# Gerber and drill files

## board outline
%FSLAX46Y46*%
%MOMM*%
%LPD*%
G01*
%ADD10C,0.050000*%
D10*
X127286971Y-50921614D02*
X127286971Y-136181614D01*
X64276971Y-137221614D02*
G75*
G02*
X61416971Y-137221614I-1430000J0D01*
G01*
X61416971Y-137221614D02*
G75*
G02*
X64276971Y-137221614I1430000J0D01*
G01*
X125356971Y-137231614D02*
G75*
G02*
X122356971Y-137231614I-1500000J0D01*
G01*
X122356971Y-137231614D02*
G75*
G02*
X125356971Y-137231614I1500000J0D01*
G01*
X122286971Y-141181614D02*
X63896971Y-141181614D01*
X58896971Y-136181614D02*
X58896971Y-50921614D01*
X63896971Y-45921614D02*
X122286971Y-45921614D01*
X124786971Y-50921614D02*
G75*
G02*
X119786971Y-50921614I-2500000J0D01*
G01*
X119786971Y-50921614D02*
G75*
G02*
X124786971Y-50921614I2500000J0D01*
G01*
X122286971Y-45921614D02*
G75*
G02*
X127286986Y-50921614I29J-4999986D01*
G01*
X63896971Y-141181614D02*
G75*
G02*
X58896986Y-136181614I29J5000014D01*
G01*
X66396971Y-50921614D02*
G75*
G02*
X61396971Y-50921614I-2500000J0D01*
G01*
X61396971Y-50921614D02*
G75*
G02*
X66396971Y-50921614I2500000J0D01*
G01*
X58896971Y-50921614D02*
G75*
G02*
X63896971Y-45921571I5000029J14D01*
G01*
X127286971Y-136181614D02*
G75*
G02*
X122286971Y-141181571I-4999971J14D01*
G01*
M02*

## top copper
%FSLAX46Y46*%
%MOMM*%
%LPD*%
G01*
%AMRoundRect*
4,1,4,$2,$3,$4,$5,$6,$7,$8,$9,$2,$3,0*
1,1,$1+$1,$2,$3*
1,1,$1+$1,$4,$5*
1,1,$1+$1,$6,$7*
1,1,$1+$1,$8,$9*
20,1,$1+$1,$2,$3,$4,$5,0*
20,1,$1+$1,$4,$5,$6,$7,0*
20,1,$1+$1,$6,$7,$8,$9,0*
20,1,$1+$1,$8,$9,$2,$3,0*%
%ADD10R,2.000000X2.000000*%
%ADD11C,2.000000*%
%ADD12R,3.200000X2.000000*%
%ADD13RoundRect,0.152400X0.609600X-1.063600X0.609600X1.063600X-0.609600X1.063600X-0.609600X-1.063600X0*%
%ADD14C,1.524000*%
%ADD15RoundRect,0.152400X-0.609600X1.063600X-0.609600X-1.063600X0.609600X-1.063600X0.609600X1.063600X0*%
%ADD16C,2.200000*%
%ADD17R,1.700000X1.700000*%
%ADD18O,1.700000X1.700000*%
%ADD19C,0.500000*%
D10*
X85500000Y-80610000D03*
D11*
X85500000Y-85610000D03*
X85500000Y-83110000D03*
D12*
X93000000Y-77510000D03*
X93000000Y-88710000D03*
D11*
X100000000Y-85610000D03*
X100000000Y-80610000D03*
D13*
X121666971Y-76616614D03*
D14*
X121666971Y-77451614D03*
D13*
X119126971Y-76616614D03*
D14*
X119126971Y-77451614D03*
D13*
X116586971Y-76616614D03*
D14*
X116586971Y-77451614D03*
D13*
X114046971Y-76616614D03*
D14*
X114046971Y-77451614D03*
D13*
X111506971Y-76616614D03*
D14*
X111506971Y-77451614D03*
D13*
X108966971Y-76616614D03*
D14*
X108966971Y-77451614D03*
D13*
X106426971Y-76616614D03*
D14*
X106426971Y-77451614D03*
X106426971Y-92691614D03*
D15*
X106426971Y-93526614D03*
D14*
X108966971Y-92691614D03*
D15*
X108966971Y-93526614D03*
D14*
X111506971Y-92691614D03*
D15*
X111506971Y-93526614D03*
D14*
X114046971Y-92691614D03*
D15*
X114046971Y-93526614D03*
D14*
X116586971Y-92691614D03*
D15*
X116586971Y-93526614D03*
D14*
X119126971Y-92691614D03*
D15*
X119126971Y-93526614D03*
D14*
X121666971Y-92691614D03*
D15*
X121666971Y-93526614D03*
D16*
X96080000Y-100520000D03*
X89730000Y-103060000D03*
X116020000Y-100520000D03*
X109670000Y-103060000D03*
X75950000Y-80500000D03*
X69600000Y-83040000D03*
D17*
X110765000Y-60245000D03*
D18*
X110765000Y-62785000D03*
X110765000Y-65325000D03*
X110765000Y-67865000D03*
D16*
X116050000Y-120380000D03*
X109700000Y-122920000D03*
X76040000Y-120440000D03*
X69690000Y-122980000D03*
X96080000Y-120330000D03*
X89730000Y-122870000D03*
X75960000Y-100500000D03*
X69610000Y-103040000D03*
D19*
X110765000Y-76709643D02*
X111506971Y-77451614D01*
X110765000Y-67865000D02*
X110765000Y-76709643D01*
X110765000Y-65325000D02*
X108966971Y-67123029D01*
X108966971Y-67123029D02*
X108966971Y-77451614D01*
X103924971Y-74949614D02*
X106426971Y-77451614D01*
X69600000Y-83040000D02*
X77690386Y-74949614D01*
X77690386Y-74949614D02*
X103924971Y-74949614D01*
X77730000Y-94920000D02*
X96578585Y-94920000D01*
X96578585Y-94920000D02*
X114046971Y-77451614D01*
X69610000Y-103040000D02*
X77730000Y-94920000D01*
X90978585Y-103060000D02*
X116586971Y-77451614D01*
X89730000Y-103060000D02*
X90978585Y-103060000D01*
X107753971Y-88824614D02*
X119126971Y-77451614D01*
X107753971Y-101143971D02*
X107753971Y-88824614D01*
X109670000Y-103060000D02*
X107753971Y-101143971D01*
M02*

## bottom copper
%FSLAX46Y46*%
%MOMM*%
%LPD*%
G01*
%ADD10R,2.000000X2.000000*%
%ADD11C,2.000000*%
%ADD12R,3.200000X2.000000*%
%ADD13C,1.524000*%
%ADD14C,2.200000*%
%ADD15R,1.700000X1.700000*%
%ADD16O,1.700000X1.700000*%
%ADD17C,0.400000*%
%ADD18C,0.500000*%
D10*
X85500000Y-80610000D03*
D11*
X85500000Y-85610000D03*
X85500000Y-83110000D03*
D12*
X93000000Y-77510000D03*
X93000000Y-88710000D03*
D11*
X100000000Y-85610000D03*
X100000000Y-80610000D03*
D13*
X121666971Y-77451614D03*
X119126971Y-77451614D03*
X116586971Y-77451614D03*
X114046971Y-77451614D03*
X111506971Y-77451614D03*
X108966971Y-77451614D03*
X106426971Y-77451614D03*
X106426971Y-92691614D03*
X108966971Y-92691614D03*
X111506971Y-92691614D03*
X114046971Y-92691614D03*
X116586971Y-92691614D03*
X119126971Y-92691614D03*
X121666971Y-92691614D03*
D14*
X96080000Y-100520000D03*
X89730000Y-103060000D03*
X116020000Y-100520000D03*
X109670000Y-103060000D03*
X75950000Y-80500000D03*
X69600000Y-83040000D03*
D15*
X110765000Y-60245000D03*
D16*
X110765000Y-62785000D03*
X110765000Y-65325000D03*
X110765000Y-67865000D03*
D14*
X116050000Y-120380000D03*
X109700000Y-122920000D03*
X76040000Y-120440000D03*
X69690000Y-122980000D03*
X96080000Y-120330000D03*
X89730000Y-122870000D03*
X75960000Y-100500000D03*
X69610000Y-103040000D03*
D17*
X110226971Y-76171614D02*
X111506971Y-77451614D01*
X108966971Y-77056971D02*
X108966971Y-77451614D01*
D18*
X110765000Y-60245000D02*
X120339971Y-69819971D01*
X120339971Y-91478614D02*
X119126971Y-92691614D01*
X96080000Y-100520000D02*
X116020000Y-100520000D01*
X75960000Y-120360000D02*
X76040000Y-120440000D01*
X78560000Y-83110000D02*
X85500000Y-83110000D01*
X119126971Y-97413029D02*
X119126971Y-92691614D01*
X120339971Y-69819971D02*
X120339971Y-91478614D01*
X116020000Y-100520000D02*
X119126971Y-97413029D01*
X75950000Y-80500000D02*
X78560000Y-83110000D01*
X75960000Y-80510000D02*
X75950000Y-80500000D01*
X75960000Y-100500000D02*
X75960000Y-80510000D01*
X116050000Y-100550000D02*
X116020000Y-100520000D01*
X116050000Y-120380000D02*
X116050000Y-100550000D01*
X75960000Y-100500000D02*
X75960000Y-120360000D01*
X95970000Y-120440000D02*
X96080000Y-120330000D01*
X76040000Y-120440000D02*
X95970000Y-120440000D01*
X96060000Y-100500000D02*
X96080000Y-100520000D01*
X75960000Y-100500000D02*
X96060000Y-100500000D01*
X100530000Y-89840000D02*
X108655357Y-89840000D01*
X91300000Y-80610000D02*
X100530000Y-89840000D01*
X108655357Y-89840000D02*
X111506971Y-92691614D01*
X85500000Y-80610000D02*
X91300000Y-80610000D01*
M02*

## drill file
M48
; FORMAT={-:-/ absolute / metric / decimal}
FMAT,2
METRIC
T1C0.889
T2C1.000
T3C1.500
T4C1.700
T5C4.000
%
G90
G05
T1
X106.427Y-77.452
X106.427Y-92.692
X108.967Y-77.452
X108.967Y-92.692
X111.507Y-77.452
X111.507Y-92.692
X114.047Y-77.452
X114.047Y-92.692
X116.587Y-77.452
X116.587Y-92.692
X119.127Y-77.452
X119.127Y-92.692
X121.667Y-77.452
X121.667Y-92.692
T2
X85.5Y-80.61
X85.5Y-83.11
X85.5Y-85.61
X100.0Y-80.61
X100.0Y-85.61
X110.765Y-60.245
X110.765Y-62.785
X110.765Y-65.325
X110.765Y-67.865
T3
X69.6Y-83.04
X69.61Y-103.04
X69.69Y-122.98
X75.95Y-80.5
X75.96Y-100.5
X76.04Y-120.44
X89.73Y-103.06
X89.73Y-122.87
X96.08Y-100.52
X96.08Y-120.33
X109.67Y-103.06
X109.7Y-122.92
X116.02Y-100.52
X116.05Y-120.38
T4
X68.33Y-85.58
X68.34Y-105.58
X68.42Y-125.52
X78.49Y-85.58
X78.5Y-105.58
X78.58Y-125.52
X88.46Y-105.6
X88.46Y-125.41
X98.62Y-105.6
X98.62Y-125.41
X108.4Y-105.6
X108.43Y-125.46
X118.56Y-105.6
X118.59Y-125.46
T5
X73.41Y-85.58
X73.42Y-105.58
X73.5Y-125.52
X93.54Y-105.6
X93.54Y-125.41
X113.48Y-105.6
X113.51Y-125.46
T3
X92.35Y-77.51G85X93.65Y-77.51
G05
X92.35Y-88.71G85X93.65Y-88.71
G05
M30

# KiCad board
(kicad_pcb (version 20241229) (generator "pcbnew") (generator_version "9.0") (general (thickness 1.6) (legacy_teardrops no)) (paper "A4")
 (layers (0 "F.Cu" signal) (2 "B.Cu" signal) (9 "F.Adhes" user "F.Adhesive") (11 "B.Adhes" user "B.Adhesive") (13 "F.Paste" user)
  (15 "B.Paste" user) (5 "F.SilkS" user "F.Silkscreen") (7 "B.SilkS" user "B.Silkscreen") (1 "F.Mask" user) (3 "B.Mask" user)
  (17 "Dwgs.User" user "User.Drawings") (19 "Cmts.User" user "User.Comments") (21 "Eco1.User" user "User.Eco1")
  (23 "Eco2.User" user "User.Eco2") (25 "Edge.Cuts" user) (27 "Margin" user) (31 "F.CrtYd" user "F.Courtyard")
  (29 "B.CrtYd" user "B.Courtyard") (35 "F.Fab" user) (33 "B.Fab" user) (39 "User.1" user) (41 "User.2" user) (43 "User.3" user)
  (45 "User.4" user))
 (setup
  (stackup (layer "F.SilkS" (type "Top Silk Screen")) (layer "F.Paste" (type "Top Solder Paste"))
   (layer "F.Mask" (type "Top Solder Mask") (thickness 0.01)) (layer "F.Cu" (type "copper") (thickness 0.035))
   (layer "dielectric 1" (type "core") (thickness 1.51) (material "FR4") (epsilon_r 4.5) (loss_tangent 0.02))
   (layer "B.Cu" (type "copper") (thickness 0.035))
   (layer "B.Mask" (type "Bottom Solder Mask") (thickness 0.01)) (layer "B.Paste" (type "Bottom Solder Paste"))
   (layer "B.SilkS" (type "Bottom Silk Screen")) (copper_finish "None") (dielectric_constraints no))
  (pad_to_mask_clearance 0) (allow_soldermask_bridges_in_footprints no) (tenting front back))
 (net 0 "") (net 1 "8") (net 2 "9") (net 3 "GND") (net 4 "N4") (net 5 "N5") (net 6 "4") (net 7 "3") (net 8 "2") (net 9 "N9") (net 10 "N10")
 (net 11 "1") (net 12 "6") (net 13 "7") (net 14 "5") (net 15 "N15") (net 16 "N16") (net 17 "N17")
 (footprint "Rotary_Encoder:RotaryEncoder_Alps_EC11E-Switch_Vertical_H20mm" (layer "F.Cu") (at 85.5 80.61)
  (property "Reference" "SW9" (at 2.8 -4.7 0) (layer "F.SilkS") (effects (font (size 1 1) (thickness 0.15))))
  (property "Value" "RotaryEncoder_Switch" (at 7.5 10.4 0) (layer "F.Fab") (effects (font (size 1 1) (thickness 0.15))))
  (pad "A" thru_hole rect (at 0 0) (size 2 2) (drill 1) (layers "*.Cu" "*.Mask") (remove_unused_layers no) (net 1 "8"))
  (pad "B" thru_hole circle (at 0 5) (size 2 2) (drill 1) (layers "*.Cu" "*.Mask") (remove_unused_layers no) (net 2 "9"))
  (pad "C" thru_hole circle (at 0 2.5) (size 2 2) (drill 1) (layers "*.Cu" "*.Mask") (remove_unused_layers no) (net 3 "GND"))
  (pad "MP" thru_hole rect (at 7.5 -3.1) (size 3.2 2) (drill oval 2.8 1.5) (layers "*.Cu" "*.Mask") (remove_unused_layers no))
  (pad "MP" thru_hole rect (at 7.5 8.1) (size 3.2 2) (drill oval 2.8 1.5) (layers "*.Cu" "*.Mask") (remove_unused_layers no))
  (pad "S1" thru_hole circle (at 14.5 5) (size 2 2) (drill 1) (layers "*.Cu" "*.Mask") (remove_unused_layers no) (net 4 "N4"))
  (pad "S2" thru_hole circle (at 14.5 0) (size 2 2) (drill 1) (layers "*.Cu" "*.Mask") (remove_unused_layers no) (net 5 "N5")))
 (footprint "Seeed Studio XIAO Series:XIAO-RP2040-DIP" (layer "F.Cu") (at 114.046971 85.071614 -90)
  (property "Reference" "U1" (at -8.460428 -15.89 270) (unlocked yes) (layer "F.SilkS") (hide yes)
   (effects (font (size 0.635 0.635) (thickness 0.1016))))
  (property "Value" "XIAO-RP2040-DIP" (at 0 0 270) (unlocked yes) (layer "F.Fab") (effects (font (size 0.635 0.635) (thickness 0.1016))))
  (pad "1" smd roundrect (at -8.455 -7.62 90) (size 2.432 1.524) (layers "F.Cu" "F.Mask") (roundrect_rratio 0.1) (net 2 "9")
   (thermal_bridge_angle 45))
  (pad "1" thru_hole circle (at -7.62 -7.62 90) (size 1.524 1.524) (drill 0.889) (layers "*.Cu" "*.Mask") (remove_unused_layers no)
   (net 2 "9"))
  (pad "2" smd roundrect (at -8.455 -5.08 90) (size 2.432 1.524) (layers "F.Cu" "F.Mask") (roundrect_rratio 0.1) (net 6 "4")
   (thermal_bridge_angle 45))
  (pad "2" thru_hole circle (at -7.62 -5.08 90) (size 1.524 1.524) (drill 0.889) (layers "*.Cu" "*.Mask") (remove_unused_layers no)
   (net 6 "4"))
  (pad "3" smd roundrect (at -8.455 -2.54 90) (size 2.432 1.524) (layers "F.Cu" "F.Mask") (roundrect_rratio 0.1) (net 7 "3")
   (thermal_bridge_angle 45))
  (pad "3" thru_hole circle (at -7.62 -2.54 90) (size 1.524 1.524) (drill 0.889) (layers "*.Cu" "*.Mask") (remove_unused_layers no)
   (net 7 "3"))
  (pad "4" smd roundrect (at -8.455 0 90) (size 2.432 1.524) (layers "F.Cu" "F.Mask") (roundrect_rratio 0.1) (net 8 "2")
   (thermal_bridge_angle 45))
  (pad "4" thru_hole circle (at -7.62 0 90) (size 1.524 1.524) (drill 0.889) (layers "*.Cu" "*.Mask") (remove_unused_layers no) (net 8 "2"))
  (pad "5" smd roundrect (at -8.455 2.54 90) (size 2.432 1.524) (layers "F.Cu" "F.Mask") (roundrect_rratio 0.1) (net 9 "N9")
   (thermal_bridge_angle 45))
  (pad "5" thru_hole circle (at -7.62 2.54 90) (size 1.524 1.524) (drill 0.889) (layers "*.Cu" "*.Mask") (remove_unused_layers no)
   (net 9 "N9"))
  (pad "6" smd roundrect (at -8.455 5.08 90) (size 2.432 1.524) (layers "F.Cu" "F.Mask") (roundrect_rratio 0.1) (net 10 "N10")
   (thermal_bridge_angle 45))
  (pad "6" thru_hole circle (at -7.62 5.08 90) (size 1.524 1.524) (drill 0.889) (layers "*.Cu" "*.Mask") (remove_unused_layers no)
   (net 10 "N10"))
  (pad "7" smd roundrect (at -8.455 7.62 90) (size 2.432 1.524) (layers "F.Cu" "F.Mask") (roundrect_rratio 0.1) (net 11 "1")
   (thermal_bridge_angle 45))
  (pad "7" thru_hole circle (at -7.62 7.62 90) (size 1.524 1.524) (drill 0.889) (layers "*.Cu" "*.Mask") (remove_unused_layers no)
   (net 11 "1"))
  (pad "8" thru_hole circle (at 7.62 7.62 270) (size 1.524 1.524) (drill 0.889) (layers "*.Cu" "*.Mask") (remove_unused_layers no)
   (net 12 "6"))
  (pad "8" smd roundrect (at 8.455 7.62 270) (size 2.432 1.524) (layers "F.Cu" "F.Mask") (roundrect_rratio 0.1) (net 12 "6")
   (thermal_bridge_angle 45))
  (pad "9" thru_hole circle (at 7.62 5.08 270) (size 1.524 1.524) (drill 0.889) (layers "*.Cu" "*.Mask") (remove_unused_layers no)
   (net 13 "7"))
  (pad "9" smd roundrect (at 8.455 5.08 270) (size 2.432 1.524) (layers "F.Cu" "F.Mask") (roundrect_rratio 0.1) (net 13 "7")
   (thermal_bridge_angle 45))
  (pad "10" thru_hole circle (at 7.62 2.54 270) (size 1.524 1.524) (drill 0.889) (layers "*.Cu" "*.Mask") (remove_unused_layers no)
   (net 1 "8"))
  (pad "10" smd roundrect (at 8.455 2.54 270) (size 2.432 1.524) (layers "F.Cu" "F.Mask") (roundrect_rratio 0.1) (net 1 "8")
   (thermal_bridge_angle 45))
  (pad "11" thru_hole circle (at 7.62 0 270) (size 1.524 1.524) (drill 0.889) (layers "*.Cu" "*.Mask") (remove_unused_layers no)
   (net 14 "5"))
  (pad "11" smd roundrect (at 8.455 0 270) (size 2.432 1.524) (layers "F.Cu" "F.Mask") (roundrect_rratio 0.1) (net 14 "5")
   (thermal_bridge_angle 45))
  (pad "12" thru_hole circle (at 7.62 -2.54 270) (size 1.524 1.524) (drill 0.889) (layers "*.Cu" "*.Mask") (remove_unused_layers no)
   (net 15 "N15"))
  (pad "12" smd roundrect (at 8.455 -2.54 270) (size 2.432 1.524) (layers "F.Cu" "F.Mask") (roundrect_rratio 0.1) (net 15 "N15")
   (thermal_bridge_angle 45))
  (pad "13" thru_hole circle (at 7.62 -5.08 270) (size 1.524 1.524) (drill 0.889) (layers "*.Cu" "*.Mask") (remove_unused_layers no)
   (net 3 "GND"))
  (pad "13" smd roundrect (at 8.455 -5.08 270) (size 2.432 1.524) (layers "F.Cu" "F.Mask") (roundrect_rratio 0.1) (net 3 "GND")
   (thermal_bridge_angle 45))
  (pad "14" thru_hole circle (at 7.62 -7.62 270) (size 1.524 1.524) (drill 0.889) (layers "*.Cu" "*.Mask") (remove_unused_layers no)
   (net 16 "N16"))
  (pad "14" smd roundrect (at 8.455 -7.62 270) (size 2.432 1.524) (layers "F.Cu" "F.Mask") (roundrect_rratio 0.1) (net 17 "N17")
   (thermal_bridge_angle 45)))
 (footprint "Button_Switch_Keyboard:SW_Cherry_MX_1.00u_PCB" (layer "F.Cu") (at 96.08 100.52)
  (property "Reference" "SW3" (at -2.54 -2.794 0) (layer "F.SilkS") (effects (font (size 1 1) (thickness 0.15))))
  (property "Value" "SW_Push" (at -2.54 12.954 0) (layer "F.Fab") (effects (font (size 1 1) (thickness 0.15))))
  (pad "" np_thru_hole circle (at -7.62 5.08) (size 1.7 1.7) (drill 1.7) (layers "*.Cu" "*.Mask"))
  (pad "" np_thru_hole circle (at -2.54 5.08) (size 4 4) (drill 4) (layers "*.Cu" "*.Mask"))
  (pad "" np_thru_hole circle (at 2.54 5.08) (size 1.7 1.7) (drill 1.7) (layers "*.Cu" "*.Mask"))
  (pad "1" thru_hole circle (at 0 0) (size 2.2 2.2) (drill 1.5) (layers "*.Cu" "*.Mask") (remove_unused_layers no) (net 3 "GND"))
  (pad "2" thru_hole circle (at -6.35 2.54) (size 2.2 2.2) (drill 1.5) (layers "*.Cu" "*.Mask") (remove_unused_layers no) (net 7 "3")))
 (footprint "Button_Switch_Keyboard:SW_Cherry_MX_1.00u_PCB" (layer "F.Cu") (at 116.02 100.52)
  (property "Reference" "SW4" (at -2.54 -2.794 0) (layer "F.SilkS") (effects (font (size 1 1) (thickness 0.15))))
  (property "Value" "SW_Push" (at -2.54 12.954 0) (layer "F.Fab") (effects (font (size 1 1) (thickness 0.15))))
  (pad "" np_thru_hole circle (at -7.62 5.08) (size 1.7 1.7) (drill 1.7) (layers "*.Cu" "*.Mask"))
  (pad "" np_thru_hole circle (at -2.54 5.08) (size 4 4) (drill 4) (layers "*.Cu" "*.Mask"))
  (pad "" np_thru_hole circle (at 2.54 5.08) (size 1.7 1.7) (drill 1.7) (layers "*.Cu" "*.Mask"))
  (pad "1" thru_hole circle (at 0 0) (size 2.2 2.2) (drill 1.5) (layers "*.Cu" "*.Mask") (remove_unused_layers no) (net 3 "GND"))
  (pad "2" thru_hole circle (at -6.35 2.54) (size 2.2 2.2) (drill 1.5) (layers "*.Cu" "*.Mask") (remove_unused_layers no) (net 6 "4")))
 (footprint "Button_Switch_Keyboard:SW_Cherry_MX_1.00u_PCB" (layer "F.Cu") (at 75.95 80.5)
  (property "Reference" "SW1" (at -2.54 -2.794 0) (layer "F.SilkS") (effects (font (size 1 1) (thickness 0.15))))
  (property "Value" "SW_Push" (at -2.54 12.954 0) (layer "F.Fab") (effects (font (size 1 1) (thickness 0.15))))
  (pad "" np_thru_hole circle (at -7.62 5.08) (size 1.7 1.7) (drill 1.7) (layers "*.Cu" "*.Mask"))
  (pad "" np_thru_hole circle (at -2.54 5.08) (size 4 4) (drill 4) (layers "*.Cu" "*.Mask"))
  (pad "" np_thru_hole circle (at 2.54 5.08) (size 1.7 1.7) (drill 1.7) (layers "*.Cu" "*.Mask"))
  (pad "1" thru_hole circle (at 0 0) (size 2.2 2.2) (drill 1.5) (layers "*.Cu" "*.Mask") (remove_unused_layers no) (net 3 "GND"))
  (pad "2" thru_hole circle (at -6.35 2.54) (size 2.2 2.2) (drill 1.5) (layers "*.Cu" "*.Mask") (remove_unused_layers no) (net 11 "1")))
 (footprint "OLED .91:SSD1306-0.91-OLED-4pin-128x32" (layer "F.Cu") (at 74.265 58.055)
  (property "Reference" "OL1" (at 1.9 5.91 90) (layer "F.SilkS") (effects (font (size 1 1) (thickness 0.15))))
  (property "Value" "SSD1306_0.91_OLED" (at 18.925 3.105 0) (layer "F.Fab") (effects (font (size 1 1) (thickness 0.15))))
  (pad "1" thru_hole rect (at 36.5 2.19) (size 1.7 1.7) (drill 1) (layers "*.Cu" "*.Mask") (remove_unused_layers no) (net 3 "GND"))
  (pad "2" thru_hole oval (at 36.5 4.73) (size 1.7 1.7) (drill 1) (layers "*.Cu" "*.Mask") (remove_unused_layers no) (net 15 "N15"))
  (pad "3" thru_hole oval (at 36.5 7.27) (size 1.7 1.7) (drill 1) (layers "*.Cu" "*.Mask") (remove_unused_layers no) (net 10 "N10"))
  (pad "4" thru_hole oval (at 36.5 9.81) (size 1.7 1.7) (drill 1) (layers "*.Cu" "*.Mask") (remove_unused_layers no) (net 9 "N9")))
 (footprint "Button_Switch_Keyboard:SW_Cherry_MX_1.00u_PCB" (layer "F.Cu") (at 116.05 120.38)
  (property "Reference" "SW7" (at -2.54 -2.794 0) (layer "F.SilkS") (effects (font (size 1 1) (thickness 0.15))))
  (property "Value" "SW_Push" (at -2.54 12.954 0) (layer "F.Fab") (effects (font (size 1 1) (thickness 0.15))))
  (pad "" np_thru_hole circle (at -7.62 5.08) (size 1.7 1.7) (drill 1.7) (layers "*.Cu" "*.Mask"))
  (pad "" np_thru_hole circle (at -2.54 5.08) (size 4 4) (drill 4) (layers "*.Cu" "*.Mask"))
  (pad "" np_thru_hole circle (at 2.54 5.08) (size 1.7 1.7) (drill 1.7) (layers "*.Cu" "*.Mask"))
  (pad "1" thru_hole circle (at 0 0) (size 2.2 2.2) (drill 1.5) (layers "*.Cu" "*.Mask") (remove_unused_layers no) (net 3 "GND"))
  (pad "2" thru_hole circle (at -6.35 2.54) (size 2.2 2.2) (drill 1.5) (layers "*.Cu" "*.Mask") (remove_unused_layers no) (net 13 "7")))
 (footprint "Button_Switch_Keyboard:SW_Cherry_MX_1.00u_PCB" (layer "F.Cu") (at 76.04 120.44)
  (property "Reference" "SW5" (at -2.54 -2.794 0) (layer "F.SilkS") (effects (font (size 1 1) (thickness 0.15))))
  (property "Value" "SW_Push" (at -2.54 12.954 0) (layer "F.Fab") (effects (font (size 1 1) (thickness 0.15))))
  (pad "" np_thru_hole circle (at -7.62 5.08) (size 1.7 1.7) (drill 1.7) (layers "*.Cu" "*.Mask"))
  (pad "" np_thru_hole circle (at -2.54 5.08) (size 4 4) (drill 4) (layers "*.Cu" "*.Mask"))
  (pad "" np_thru_hole circle (at 2.54 5.08) (size 1.7 1.7) (drill 1.7) (layers "*.Cu" "*.Mask"))
  (pad "1" thru_hole circle (at 0 0) (size 2.2 2.2) (drill 1.5) (layers "*.Cu" "*.Mask") (remove_unused_layers no) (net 3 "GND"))
  (pad "2" thru_hole circle (at -6.35 2.54) (size 2.2 2.2) (drill 1.5) (layers "*.Cu" "*.Mask") (remove_unused_layers no) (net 14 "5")))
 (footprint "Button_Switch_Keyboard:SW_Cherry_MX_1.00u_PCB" (layer "F.Cu") (at 96.08 120.33)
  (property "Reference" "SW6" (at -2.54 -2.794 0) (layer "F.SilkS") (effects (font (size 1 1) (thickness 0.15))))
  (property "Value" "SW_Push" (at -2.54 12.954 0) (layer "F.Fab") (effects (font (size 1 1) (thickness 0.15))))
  (pad "" np_thru_hole circle (at -7.62 5.08) (size 1.7 1.7) (drill 1.7) (layers "*.Cu" "*.Mask"))
  (pad "" np_thru_hole circle (at -2.54 5.08) (size 4 4) (drill 4) (layers "*.Cu" "*.Mask"))
  (pad "" np_thru_hole circle (at 2.54 5.08) (size 1.7 1.7) (drill 1.7) (layers "*.Cu" "*.Mask"))
  (pad "1" thru_hole circle (at 0 0) (size 2.2 2.2) (drill 1.5) (layers "*.Cu" "*.Mask") (remove_unused_layers no) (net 3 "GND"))
  (pad "2" thru_hole circle (at -6.35 2.54) (size 2.2 2.2) (drill 1.5) (layers "*.Cu" "*.Mask") (remove_unused_layers no) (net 12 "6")))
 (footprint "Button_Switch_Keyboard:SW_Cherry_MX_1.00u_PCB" (layer "F.Cu") (at 75.96 100.5)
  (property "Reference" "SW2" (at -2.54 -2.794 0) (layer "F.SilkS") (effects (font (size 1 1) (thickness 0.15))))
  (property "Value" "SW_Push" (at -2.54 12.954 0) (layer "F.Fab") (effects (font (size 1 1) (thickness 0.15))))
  (pad "" np_thru_hole circle (at -7.62 5.08) (size 1.7 1.7) (drill 1.7) (layers "*.Cu" "*.Mask"))
  (pad "" np_thru_hole circle (at -2.54 5.08) (size 4 4) (drill 4) (layers "*.Cu" "*.Mask"))
  (pad "" np_thru_hole circle (at 2.54 5.08) (size 1.7 1.7) (drill 1.7) (layers "*.Cu" "*.Mask"))
  (pad "1" thru_hole circle (at 0 0) (size 2.2 2.2) (drill 1.5) (layers "*.Cu" "*.Mask") (remove_unused_layers no) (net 3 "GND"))
  (pad "2" thru_hole circle (at -6.35 2.54) (size 2.2 2.2) (drill 1.5) (layers "*.Cu" "*.Mask") (remove_unused_layers no) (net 8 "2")))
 (gr_line (start 127.286971 50.921614) (end 127.286971 136.181614) (stroke (width 0.05) (type default)) (layer "Edge.Cuts"))
 (gr_circle (center 62.846971 137.221614) (end 64.276971 137.221614) (stroke (width 0.05) (type solid)) (fill no) (layer "Edge.Cuts"))
 (gr_circle (center 123.856971 137.231614) (end 125.356971 137.231614) (stroke (width 0.05) (type solid)) (fill no) (layer "Edge.Cuts"))
 (gr_line (start 122.286971 141.181614) (end 63.896971 141.181614) (stroke (width 0.05) (type default)) (layer "Edge.Cuts"))
 (gr_line (start 58.896971 136.181614) (end 58.896971 50.921614) (stroke (width 0.05) (type default)) (layer "Edge.Cuts"))
 (gr_line (start 63.896971 45.921614) (end 122.286971 45.921614) (stroke (width 0.05) (type default)) (layer "Edge.Cuts"))
 (gr_circle (center 122.286971 50.921614) (end 124.786971 50.921614) (stroke (width 0.05) (type solid)) (fill no) (layer "Edge.Cuts"))
 (gr_arc (start 122.286971 45.921614) (mid 125.822505 47.38608) (end 127.286971 50.921614) (stroke (width 0.05) (type default))
  (layer "Edge.Cuts"))
 (gr_arc (start 63.896971 141.181614) (mid 60.361437 139.717148) (end 58.896971 136.181614) (stroke (width 0.05) (type default))
  (layer "Edge.Cuts"))
 (gr_circle (center 63.896971 50.921614) (end 66.396971 50.921614) (stroke (width 0.05) (type solid)) (fill no) (layer "Edge.Cuts"))
 (gr_arc (start 58.896971 50.921614) (mid 60.361437 47.38608) (end 63.896971 45.921614) (stroke (width 0.05) (type default))
  (layer "Edge.Cuts"))
 (gr_arc (start 127.286971 136.181614) (mid 125.822505 139.717148) (end 122.286971 141.181614) (stroke (width 0.05) (type default))
  (layer "Edge.Cuts"))
 (segment (start 110.765 76.709643) (end 111.506971 77.451614) (width 0.5) (layer "F.Cu") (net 9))
 (segment (start 110.765 67.865) (end 110.765 76.709643) (width 0.5) (layer "F.Cu") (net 9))
 (segment (start 110.226971 76.171614) (end 111.506971 77.451614) (width 0.4) (layer "B.Cu") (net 9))
 (segment (start 110.765 65.325) (end 108.966971 67.123029) (width 0.5) (layer "F.Cu") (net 10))
 (segment (start 108.966971 67.123029) (end 108.966971 77.451614) (width 0.5) (layer "F.Cu") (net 10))
 (segment (start 108.966971 77.056971) (end 108.966971 77.451614) (width 0.4) (layer "B.Cu") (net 10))
 (segment (start 110.765 60.245) (end 120.339971 69.819971) (width 0.5) (layer "B.Cu") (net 3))
 (segment (start 120.339971 91.478614) (end 119.126971 92.691614) (width 0.5) (layer "B.Cu") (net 3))
 (segment (start 96.08 100.52) (end 116.02 100.52) (width 0.5) (layer "B.Cu") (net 3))
 (segment (start 75.96 120.36) (end 76.04 120.44) (width 0.5) (layer "B.Cu") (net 3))
 (segment (start 78.56 83.11) (end 85.5 83.11) (width 0.5) (layer "B.Cu") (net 3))
 (segment (start 119.126971 97.413029) (end 119.126971 92.691614) (width 0.5) (layer "B.Cu") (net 3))
 (segment (start 120.339971 69.819971) (end 120.339971 91.478614) (width 0.5) (layer "B.Cu") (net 3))
 (segment (start 116.02 100.52) (end 119.126971 97.413029) (width 0.5) (layer "B.Cu") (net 3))
 (segment (start 75.95 80.5) (end 78.56 83.11) (width 0.5) (layer "B.Cu") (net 3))
 (segment (start 75.96 80.51) (end 75.95 80.5) (width 0.5) (layer "B.Cu") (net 3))
 (segment (start 75.96 100.5) (end 75.96 80.51) (width 0.5) (layer "B.Cu") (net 3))
 (segment (start 116.05 100.55) (end 116.02 100.52) (width 0.5) (layer "B.Cu") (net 3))
 (segment (start 116.05 120.38) (end 116.05 100.55) (width 0.5) (layer "B.Cu") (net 3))
 (segment (start 75.96 100.5) (end 75.96 120.36) (width 0.5) (layer "B.Cu") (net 3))
 (segment (start 95.97 120.44) (end 96.08 120.33) (width 0.5) (layer "B.Cu") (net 3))
 (segment (start 76.04 120.44) (end 95.97 120.44) (width 0.5) (layer "B.Cu") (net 3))
 (segment (start 96.06 100.5) (end 96.08 100.52) (width 0.5) (layer "B.Cu") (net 3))
 (segment (start 75.96 100.5) (end 96.06 100.5) (width 0.5) (layer "B.Cu") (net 3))
 (segment (start 103.924971 74.949614) (end 106.426971 77.451614) (width 0.5) (layer "F.Cu") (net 11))
 (segment (start 69.6 83.04) (end 77.690386 74.949614) (width 0.5) (layer "F.Cu") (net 11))
 (segment (start 77.690386 74.949614) (end 103.924971 74.949614) (width 0.5) (layer "F.Cu") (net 11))
 (segment (start 77.73 94.92) (end 96.578585 94.92) (width 0.5) (layer "F.Cu") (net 8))
 (segment (start 96.578585 94.92) (end 114.046971 77.451614) (width 0.5) (layer "F.Cu") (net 8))
 (segment (start 69.61 103.04) (end 77.73 94.92) (width 0.5) (layer "F.Cu") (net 8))
 (segment (start 90.978585 103.06) (end 116.586971 77.451614) (width 0.5) (layer "F.Cu") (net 7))
 (segment (start 89.73 103.06) (end 90.978585 103.06) (width 0.5) (layer "F.Cu") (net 7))
 (segment (start 107.753971 88.824614) (end 119.126971 77.451614) (width 0.5) (layer "F.Cu") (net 6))
 (segment (start 107.753971 101.143971) (end 107.753971 88.824614) (width 0.5) (layer "F.Cu") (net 6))
 (segment (start 109.67 103.06) (end 107.753971 101.143971) (width 0.5) (layer "F.Cu") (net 6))
 (segment (start 100.53 89.84) (end 108.655357 89.84) (width 0.5) (layer "B.Cu") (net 1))
 (segment (start 91.3 80.61) (end 100.53 89.84) (width 0.5) (layer "B.Cu") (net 1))
 (segment (start 108.655357 89.84) (end 111.506971 92.691614) (width 0.5) (layer "B.Cu") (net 1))
 (segment (start 85.5 80.61) (end 91.3 80.61) (width 0.5) (layer "B.Cu") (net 1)))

